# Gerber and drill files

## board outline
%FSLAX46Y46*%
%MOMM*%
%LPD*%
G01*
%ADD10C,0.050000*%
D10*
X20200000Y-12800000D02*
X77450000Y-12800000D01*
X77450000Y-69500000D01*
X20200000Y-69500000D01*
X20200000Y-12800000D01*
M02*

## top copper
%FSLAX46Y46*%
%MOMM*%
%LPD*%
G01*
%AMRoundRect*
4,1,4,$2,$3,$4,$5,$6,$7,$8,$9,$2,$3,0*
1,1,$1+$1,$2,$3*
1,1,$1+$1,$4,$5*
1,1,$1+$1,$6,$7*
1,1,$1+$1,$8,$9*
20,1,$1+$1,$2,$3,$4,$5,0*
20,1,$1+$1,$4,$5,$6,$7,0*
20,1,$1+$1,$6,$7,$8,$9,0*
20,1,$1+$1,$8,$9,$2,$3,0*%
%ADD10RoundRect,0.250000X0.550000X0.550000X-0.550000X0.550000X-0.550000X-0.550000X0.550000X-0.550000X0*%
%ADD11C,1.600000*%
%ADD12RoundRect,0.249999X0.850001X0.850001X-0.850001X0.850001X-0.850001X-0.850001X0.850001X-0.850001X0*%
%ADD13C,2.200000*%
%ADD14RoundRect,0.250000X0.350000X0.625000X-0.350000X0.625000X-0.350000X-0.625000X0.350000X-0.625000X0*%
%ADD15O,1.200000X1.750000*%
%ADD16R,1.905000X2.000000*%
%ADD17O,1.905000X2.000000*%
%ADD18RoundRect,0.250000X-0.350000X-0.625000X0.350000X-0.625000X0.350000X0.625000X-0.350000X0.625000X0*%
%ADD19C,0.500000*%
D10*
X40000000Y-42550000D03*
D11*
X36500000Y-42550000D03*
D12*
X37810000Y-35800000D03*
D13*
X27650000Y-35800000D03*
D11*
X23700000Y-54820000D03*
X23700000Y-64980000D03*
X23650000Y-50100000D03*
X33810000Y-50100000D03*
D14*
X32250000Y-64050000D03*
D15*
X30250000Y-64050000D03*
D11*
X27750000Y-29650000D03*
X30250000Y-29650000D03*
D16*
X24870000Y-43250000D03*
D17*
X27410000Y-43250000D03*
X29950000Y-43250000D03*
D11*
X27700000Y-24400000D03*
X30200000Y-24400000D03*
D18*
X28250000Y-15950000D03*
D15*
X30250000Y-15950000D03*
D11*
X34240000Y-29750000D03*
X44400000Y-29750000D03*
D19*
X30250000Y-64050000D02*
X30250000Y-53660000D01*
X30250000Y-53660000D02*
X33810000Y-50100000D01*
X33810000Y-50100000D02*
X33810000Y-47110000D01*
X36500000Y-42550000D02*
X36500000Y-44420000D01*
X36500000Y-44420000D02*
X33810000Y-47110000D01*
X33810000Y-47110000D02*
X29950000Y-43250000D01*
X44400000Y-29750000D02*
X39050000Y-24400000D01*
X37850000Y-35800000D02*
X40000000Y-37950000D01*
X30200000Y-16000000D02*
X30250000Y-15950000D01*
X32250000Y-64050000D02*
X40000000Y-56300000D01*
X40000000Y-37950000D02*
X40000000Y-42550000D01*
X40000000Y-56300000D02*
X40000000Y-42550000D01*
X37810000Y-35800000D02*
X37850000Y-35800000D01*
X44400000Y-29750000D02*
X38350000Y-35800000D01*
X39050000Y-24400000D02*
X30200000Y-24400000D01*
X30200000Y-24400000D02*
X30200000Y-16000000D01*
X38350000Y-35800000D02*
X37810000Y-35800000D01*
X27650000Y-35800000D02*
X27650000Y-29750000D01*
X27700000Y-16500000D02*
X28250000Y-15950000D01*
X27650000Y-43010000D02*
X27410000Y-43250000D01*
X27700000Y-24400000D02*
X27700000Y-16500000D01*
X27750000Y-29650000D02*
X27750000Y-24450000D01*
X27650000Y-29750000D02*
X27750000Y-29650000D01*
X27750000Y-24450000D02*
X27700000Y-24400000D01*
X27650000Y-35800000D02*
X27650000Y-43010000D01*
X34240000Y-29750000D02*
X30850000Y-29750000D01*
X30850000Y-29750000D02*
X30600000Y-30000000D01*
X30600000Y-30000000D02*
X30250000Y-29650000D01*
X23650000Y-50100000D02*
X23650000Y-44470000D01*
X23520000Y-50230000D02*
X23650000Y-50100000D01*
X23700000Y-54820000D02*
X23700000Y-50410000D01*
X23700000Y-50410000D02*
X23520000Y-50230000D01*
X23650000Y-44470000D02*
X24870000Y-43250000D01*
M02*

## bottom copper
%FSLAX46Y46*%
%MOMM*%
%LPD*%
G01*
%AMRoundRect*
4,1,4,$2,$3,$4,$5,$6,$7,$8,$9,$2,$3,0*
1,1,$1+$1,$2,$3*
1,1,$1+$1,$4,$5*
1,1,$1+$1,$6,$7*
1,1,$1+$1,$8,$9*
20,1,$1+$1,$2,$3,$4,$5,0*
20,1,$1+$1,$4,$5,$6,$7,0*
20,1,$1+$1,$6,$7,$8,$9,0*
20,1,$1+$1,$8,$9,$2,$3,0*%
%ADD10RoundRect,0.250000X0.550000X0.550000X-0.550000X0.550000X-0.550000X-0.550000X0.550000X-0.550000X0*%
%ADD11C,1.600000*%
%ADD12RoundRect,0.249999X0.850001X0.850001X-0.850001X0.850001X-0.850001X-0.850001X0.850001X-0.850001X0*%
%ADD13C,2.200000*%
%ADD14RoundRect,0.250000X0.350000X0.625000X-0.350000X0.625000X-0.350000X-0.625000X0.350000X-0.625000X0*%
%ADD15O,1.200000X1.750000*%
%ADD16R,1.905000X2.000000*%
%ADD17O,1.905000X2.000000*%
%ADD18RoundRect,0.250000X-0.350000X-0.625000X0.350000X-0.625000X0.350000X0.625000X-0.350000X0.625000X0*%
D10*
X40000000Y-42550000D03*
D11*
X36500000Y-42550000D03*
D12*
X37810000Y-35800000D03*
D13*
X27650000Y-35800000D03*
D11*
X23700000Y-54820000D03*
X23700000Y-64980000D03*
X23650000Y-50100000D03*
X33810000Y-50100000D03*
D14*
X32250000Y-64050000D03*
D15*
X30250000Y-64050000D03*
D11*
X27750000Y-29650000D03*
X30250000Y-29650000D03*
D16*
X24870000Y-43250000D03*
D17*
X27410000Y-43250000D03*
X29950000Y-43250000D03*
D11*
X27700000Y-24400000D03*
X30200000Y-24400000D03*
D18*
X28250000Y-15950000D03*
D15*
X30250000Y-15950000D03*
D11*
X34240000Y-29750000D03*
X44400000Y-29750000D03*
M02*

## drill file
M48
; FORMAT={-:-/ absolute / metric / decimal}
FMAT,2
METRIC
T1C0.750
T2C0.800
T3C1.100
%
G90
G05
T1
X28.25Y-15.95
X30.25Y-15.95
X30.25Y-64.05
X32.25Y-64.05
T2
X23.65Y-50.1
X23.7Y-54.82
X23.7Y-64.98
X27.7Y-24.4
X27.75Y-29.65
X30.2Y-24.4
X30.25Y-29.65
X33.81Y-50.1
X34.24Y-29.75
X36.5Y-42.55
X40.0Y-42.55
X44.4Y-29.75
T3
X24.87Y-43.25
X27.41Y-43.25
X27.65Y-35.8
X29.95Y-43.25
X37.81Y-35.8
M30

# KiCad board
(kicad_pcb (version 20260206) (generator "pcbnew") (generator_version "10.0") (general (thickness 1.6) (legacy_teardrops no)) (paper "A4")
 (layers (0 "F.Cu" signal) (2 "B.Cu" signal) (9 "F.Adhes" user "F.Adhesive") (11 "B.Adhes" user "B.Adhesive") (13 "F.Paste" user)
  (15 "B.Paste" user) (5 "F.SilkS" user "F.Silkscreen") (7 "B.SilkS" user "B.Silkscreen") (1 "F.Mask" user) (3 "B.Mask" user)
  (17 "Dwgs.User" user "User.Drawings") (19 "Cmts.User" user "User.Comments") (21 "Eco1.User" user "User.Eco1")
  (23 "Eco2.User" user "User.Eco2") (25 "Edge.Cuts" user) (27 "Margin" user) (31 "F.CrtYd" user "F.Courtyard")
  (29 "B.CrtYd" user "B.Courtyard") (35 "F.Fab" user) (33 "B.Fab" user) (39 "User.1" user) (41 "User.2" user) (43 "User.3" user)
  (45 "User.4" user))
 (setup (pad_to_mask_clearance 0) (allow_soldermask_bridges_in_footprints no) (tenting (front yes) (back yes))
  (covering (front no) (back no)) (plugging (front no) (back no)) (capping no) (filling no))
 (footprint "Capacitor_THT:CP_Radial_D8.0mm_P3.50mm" (layer "F.Cu") (at 40 42.55 180)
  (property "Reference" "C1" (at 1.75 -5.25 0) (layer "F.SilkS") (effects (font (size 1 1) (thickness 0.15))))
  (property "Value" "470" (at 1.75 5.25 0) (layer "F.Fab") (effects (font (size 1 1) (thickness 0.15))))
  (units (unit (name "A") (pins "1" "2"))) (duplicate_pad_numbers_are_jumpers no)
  (pad "1" thru_hole roundrect (at 0 0 180) (size 1.6 1.6) (drill 0.8) (layers "*.Cu" "*.Mask") (remove_unused_layers no)
   (roundrect_rratio 0.15625) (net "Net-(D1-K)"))
  (pad "2" thru_hole circle (at 3.5 0 180) (size 1.6 1.6) (drill 0.8) (layers "*.Cu" "*.Mask") (remove_unused_layers no)
   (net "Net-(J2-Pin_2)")))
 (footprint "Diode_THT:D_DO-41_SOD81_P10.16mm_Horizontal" (layer "F.Cu") (at 37.81 35.8 180)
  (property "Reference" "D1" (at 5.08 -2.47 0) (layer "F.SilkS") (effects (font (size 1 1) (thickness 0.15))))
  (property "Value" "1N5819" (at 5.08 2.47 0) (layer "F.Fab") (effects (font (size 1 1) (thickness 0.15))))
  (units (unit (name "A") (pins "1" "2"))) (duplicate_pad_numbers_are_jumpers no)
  (pad "1" thru_hole roundrect (at 0 0 180) (size 2.2 2.2) (drill 1.1) (layers "*.Cu" "*.Mask") (remove_unused_layers no)
   (roundrect_rratio 0.113636) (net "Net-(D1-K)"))
  (pad "2" thru_hole circle (at 10.16 0 180) (size 2.2 2.2) (drill 1.1) (layers "*.Cu" "*.Mask") (remove_unused_layers no)
   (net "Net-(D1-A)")))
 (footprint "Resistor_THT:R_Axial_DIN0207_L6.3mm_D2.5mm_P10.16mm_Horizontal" (layer "F.Cu") (at 23.7 54.82 -90)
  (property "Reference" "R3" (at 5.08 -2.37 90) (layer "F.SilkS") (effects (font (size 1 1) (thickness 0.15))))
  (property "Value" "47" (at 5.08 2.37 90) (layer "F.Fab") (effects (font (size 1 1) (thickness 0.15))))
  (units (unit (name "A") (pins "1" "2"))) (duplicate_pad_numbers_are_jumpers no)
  (pad "1" thru_hole circle (at 0 0 270) (size 1.6 1.6) (drill 0.8) (layers "*.Cu" "*.Mask") (remove_unused_layers no) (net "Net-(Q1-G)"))
  (pad "2" thru_hole circle (at 10.16 0 270) (size 1.6 1.6) (drill 0.8) (layers "*.Cu" "*.Mask") (remove_unused_layers no) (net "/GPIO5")))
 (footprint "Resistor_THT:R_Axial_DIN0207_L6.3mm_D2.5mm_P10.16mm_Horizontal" (layer "F.Cu") (at 23.65 50.1)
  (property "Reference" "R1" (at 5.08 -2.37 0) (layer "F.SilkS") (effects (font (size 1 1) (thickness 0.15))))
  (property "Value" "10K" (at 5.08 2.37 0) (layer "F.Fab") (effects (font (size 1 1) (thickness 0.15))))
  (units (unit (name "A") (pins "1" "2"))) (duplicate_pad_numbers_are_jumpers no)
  (pad "1" thru_hole circle (at 0 0) (size 1.6 1.6) (drill 0.8) (layers "*.Cu" "*.Mask") (remove_unused_layers no) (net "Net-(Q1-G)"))
  (pad "2" thru_hole circle (at 10.16 0) (size 1.6 1.6) (drill 0.8) (layers "*.Cu" "*.Mask") (remove_unused_layers no)
   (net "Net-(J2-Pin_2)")))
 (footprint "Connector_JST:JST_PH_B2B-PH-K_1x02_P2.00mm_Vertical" (layer "F.Cu") (at 32.25 64.05 180)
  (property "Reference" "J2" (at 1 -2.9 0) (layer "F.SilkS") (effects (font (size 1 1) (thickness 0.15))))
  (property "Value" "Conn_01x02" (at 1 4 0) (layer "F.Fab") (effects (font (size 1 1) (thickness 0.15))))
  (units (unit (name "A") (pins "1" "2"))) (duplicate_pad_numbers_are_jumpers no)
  (pad "1" thru_hole roundrect (at 0 0 180) (size 1.2 1.75) (drill 0.75) (layers "*.Cu" "*.Mask") (remove_unused_layers no)
   (roundrect_rratio 0.208333) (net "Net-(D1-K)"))
  (pad "2" thru_hole oval (at 2 0 180) (size 1.2 1.75) (drill 0.75) (layers "*.Cu" "*.Mask") (remove_unused_layers no)
   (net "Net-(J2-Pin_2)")))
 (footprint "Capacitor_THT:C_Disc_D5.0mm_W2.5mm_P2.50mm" (layer "F.Cu") (at 27.75 29.65)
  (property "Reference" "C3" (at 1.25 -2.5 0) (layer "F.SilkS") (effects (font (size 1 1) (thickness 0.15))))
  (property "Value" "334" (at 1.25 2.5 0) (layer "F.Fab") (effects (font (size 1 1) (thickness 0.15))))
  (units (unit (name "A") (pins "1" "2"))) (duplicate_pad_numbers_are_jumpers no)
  (pad "1" thru_hole circle (at 0 0) (size 1.6 1.6) (drill 0.8) (layers "*.Cu" "*.Mask") (remove_unused_layers no) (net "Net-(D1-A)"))
  (pad "2" thru_hole circle (at 2.5 0) (size 1.6 1.6) (drill 0.8) (layers "*.Cu" "*.Mask") (remove_unused_layers no) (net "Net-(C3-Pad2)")))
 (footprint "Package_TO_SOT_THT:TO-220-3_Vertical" (layer "F.Cu") (at 24.87 43.25)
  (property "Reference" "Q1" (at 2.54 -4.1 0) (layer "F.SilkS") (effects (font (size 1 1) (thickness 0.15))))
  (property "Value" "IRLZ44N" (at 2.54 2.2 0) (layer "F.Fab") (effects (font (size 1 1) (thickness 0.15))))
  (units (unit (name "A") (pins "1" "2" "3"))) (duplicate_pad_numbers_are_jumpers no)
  (pad "1" thru_hole rect (at 0 0) (size 1.905 2) (drill 1.1) (layers "*.Cu" "*.Mask") (remove_unused_layers no) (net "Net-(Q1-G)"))
  (pad "2" thru_hole oval (at 2.54 0) (size 1.905 2) (drill 1.1) (layers "*.Cu" "*.Mask") (remove_unused_layers no) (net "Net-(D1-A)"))
  (pad "3" thru_hole oval (at 5.08 0) (size 1.905 2) (drill 1.1) (layers "*.Cu" "*.Mask") (remove_unused_layers no) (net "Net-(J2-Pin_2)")))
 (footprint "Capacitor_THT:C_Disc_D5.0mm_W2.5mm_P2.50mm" (layer "F.Cu") (at 27.7 24.4)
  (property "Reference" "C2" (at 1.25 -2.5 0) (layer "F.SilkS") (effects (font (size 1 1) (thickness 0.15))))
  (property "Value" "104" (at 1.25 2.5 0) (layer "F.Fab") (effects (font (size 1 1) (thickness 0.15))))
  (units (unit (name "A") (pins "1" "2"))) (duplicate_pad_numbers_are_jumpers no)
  (pad "1" thru_hole circle (at 0 0) (size 1.6 1.6) (drill 0.8) (layers "*.Cu" "*.Mask") (remove_unused_layers no) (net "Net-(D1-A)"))
  (pad "2" thru_hole circle (at 2.5 0) (size 1.6 1.6) (drill 0.8) (layers "*.Cu" "*.Mask") (remove_unused_layers no) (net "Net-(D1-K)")))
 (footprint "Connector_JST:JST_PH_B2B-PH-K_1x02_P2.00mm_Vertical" (layer "F.Cu") (at 28.25 15.95)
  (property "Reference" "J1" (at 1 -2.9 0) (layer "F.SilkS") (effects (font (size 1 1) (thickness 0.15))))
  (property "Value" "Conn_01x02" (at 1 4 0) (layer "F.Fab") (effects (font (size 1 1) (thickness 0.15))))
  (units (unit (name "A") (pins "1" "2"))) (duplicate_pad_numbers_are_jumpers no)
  (pad "1" thru_hole roundrect (at 0 0) (size 1.2 1.75) (drill 0.75) (layers "*.Cu" "*.Mask") (remove_unused_layers no)
   (roundrect_rratio 0.208333) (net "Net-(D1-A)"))
  (pad "2" thru_hole oval (at 2 0) (size 1.2 1.75) (drill 0.75) (layers "*.Cu" "*.Mask") (remove_unused_layers no) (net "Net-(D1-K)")))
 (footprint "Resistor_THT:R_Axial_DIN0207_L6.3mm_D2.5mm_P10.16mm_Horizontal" (layer "F.Cu") (at 34.24 29.75)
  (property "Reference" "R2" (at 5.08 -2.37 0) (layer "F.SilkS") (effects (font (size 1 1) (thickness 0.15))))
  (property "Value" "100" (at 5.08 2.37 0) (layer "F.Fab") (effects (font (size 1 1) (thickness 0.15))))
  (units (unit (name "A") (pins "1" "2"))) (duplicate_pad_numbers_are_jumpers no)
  (pad "1" thru_hole circle (at 0 0) (size 1.6 1.6) (drill 0.8) (layers "*.Cu" "*.Mask") (remove_unused_layers no) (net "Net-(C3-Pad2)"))
  (pad "2" thru_hole circle (at 10.16 0) (size 1.6 1.6) (drill 0.8) (layers "*.Cu" "*.Mask") (remove_unused_layers no) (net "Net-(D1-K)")))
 (gr_rect (start 20.2 12.8) (end 77.45 69.5) (stroke (width 0.05) (type default)) (fill no) (layer "Edge.Cuts"))
 (segment (start 30.25 64.05) (end 30.25 53.66) (width 0.5) (layer "F.Cu") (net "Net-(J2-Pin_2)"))
 (segment (start 30.25 53.66) (end 33.81 50.1) (width 0.5) (layer "F.Cu") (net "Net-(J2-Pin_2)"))
 (segment (start 33.81 50.1) (end 33.81 47.11) (width 0.5) (layer "F.Cu") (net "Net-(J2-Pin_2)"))
 (segment (start 36.5 42.55) (end 36.5 44.42) (width 0.5) (layer "F.Cu") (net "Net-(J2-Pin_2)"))
 (segment (start 36.5 44.42) (end 33.81 47.11) (width 0.5) (layer "F.Cu") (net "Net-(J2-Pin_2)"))
 (segment (start 33.81 47.11) (end 29.95 43.25) (width 0.5) (layer "F.Cu") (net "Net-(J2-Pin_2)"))
 (segment (start 44.4 29.75) (end 39.05 24.4) (width 0.5) (layer "F.Cu") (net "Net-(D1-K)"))
 (segment (start 37.85 35.8) (end 40 37.95) (width 0.5) (layer "F.Cu") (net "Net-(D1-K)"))
 (segment (start 30.2 16) (end 30.25 15.95) (width 0.5) (layer "F.Cu") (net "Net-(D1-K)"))
 (segment (start 32.25 64.05) (end 40 56.3) (width 0.5) (layer "F.Cu") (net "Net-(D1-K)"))
 (segment (start 40 37.95) (end 40 42.55) (width 0.5) (layer "F.Cu") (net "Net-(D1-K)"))
 (segment (start 40 56.3) (end 40 42.55) (width 0.5) (layer "F.Cu") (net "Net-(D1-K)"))
 (segment (start 37.81 35.8) (end 37.85 35.8) (width 0.5) (layer "F.Cu") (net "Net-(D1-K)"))
 (segment (start 44.4 29.75) (end 38.35 35.8) (width 0.5) (layer "F.Cu") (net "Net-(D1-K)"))
 (segment (start 39.05 24.4) (end 30.2 24.4) (width 0.5) (layer "F.Cu") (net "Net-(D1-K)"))
 (segment (start 30.2 24.4) (end 30.2 16) (width 0.5) (layer "F.Cu") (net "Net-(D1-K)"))
 (segment (start 38.35 35.8) (end 37.81 35.8) (width 0.5) (layer "F.Cu") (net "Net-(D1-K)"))
 (segment (start 27.65 35.8) (end 27.65 29.75) (width 0.5) (layer "F.Cu") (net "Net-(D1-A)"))
 (segment (start 27.7 16.5) (end 28.25 15.95) (width 0.5) (layer "F.Cu") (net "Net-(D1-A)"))
 (segment (start 27.65 43.01) (end 27.41 43.25) (width 0.5) (layer "F.Cu") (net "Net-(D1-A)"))
 (segment (start 27.7 24.4) (end 27.7 16.5) (width 0.5) (layer "F.Cu") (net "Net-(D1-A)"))
 (segment (start 27.75 29.65) (end 27.75 24.45) (width 0.5) (layer "F.Cu") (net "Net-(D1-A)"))
 (segment (start 27.65 29.75) (end 27.75 29.65) (width 0.5) (layer "F.Cu") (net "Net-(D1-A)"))
 (segment (start 27.75 24.45) (end 27.7 24.4) (width 0.5) (layer "F.Cu") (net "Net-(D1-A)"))
 (segment (start 27.65 35.8) (end 27.65 43.01) (width 0.5) (layer "F.Cu") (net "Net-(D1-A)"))
 (segment (start 34.24 29.75) (end 30.85 29.75) (width 0.5) (layer "F.Cu") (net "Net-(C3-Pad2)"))
 (segment (start 30.85 29.75) (end 30.6 30) (width 0.5) (layer "F.Cu") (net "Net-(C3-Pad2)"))
 (segment (start 30.6 30) (end 30.25 29.65) (width 0.5) (layer "F.Cu") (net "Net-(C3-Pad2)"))
 (segment (start 23.65 50.1) (end 23.65 44.47) (width 0.5) (layer "F.Cu") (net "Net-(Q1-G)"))
 (segment (start 23.52 50.23) (end 23.65 50.1) (width 0.5) (layer "F.Cu") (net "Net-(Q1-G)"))
 (segment (start 23.7 54.82) (end 23.7 50.41) (width 0.5) (layer "F.Cu") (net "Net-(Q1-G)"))
 (segment (start 23.7 50.41) (end 23.52 50.23) (width 0.5) (layer "F.Cu") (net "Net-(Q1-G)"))
 (segment (start 23.65 44.47) (end 24.87 43.25) (width 0.5) (layer "F.Cu") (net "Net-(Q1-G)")))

